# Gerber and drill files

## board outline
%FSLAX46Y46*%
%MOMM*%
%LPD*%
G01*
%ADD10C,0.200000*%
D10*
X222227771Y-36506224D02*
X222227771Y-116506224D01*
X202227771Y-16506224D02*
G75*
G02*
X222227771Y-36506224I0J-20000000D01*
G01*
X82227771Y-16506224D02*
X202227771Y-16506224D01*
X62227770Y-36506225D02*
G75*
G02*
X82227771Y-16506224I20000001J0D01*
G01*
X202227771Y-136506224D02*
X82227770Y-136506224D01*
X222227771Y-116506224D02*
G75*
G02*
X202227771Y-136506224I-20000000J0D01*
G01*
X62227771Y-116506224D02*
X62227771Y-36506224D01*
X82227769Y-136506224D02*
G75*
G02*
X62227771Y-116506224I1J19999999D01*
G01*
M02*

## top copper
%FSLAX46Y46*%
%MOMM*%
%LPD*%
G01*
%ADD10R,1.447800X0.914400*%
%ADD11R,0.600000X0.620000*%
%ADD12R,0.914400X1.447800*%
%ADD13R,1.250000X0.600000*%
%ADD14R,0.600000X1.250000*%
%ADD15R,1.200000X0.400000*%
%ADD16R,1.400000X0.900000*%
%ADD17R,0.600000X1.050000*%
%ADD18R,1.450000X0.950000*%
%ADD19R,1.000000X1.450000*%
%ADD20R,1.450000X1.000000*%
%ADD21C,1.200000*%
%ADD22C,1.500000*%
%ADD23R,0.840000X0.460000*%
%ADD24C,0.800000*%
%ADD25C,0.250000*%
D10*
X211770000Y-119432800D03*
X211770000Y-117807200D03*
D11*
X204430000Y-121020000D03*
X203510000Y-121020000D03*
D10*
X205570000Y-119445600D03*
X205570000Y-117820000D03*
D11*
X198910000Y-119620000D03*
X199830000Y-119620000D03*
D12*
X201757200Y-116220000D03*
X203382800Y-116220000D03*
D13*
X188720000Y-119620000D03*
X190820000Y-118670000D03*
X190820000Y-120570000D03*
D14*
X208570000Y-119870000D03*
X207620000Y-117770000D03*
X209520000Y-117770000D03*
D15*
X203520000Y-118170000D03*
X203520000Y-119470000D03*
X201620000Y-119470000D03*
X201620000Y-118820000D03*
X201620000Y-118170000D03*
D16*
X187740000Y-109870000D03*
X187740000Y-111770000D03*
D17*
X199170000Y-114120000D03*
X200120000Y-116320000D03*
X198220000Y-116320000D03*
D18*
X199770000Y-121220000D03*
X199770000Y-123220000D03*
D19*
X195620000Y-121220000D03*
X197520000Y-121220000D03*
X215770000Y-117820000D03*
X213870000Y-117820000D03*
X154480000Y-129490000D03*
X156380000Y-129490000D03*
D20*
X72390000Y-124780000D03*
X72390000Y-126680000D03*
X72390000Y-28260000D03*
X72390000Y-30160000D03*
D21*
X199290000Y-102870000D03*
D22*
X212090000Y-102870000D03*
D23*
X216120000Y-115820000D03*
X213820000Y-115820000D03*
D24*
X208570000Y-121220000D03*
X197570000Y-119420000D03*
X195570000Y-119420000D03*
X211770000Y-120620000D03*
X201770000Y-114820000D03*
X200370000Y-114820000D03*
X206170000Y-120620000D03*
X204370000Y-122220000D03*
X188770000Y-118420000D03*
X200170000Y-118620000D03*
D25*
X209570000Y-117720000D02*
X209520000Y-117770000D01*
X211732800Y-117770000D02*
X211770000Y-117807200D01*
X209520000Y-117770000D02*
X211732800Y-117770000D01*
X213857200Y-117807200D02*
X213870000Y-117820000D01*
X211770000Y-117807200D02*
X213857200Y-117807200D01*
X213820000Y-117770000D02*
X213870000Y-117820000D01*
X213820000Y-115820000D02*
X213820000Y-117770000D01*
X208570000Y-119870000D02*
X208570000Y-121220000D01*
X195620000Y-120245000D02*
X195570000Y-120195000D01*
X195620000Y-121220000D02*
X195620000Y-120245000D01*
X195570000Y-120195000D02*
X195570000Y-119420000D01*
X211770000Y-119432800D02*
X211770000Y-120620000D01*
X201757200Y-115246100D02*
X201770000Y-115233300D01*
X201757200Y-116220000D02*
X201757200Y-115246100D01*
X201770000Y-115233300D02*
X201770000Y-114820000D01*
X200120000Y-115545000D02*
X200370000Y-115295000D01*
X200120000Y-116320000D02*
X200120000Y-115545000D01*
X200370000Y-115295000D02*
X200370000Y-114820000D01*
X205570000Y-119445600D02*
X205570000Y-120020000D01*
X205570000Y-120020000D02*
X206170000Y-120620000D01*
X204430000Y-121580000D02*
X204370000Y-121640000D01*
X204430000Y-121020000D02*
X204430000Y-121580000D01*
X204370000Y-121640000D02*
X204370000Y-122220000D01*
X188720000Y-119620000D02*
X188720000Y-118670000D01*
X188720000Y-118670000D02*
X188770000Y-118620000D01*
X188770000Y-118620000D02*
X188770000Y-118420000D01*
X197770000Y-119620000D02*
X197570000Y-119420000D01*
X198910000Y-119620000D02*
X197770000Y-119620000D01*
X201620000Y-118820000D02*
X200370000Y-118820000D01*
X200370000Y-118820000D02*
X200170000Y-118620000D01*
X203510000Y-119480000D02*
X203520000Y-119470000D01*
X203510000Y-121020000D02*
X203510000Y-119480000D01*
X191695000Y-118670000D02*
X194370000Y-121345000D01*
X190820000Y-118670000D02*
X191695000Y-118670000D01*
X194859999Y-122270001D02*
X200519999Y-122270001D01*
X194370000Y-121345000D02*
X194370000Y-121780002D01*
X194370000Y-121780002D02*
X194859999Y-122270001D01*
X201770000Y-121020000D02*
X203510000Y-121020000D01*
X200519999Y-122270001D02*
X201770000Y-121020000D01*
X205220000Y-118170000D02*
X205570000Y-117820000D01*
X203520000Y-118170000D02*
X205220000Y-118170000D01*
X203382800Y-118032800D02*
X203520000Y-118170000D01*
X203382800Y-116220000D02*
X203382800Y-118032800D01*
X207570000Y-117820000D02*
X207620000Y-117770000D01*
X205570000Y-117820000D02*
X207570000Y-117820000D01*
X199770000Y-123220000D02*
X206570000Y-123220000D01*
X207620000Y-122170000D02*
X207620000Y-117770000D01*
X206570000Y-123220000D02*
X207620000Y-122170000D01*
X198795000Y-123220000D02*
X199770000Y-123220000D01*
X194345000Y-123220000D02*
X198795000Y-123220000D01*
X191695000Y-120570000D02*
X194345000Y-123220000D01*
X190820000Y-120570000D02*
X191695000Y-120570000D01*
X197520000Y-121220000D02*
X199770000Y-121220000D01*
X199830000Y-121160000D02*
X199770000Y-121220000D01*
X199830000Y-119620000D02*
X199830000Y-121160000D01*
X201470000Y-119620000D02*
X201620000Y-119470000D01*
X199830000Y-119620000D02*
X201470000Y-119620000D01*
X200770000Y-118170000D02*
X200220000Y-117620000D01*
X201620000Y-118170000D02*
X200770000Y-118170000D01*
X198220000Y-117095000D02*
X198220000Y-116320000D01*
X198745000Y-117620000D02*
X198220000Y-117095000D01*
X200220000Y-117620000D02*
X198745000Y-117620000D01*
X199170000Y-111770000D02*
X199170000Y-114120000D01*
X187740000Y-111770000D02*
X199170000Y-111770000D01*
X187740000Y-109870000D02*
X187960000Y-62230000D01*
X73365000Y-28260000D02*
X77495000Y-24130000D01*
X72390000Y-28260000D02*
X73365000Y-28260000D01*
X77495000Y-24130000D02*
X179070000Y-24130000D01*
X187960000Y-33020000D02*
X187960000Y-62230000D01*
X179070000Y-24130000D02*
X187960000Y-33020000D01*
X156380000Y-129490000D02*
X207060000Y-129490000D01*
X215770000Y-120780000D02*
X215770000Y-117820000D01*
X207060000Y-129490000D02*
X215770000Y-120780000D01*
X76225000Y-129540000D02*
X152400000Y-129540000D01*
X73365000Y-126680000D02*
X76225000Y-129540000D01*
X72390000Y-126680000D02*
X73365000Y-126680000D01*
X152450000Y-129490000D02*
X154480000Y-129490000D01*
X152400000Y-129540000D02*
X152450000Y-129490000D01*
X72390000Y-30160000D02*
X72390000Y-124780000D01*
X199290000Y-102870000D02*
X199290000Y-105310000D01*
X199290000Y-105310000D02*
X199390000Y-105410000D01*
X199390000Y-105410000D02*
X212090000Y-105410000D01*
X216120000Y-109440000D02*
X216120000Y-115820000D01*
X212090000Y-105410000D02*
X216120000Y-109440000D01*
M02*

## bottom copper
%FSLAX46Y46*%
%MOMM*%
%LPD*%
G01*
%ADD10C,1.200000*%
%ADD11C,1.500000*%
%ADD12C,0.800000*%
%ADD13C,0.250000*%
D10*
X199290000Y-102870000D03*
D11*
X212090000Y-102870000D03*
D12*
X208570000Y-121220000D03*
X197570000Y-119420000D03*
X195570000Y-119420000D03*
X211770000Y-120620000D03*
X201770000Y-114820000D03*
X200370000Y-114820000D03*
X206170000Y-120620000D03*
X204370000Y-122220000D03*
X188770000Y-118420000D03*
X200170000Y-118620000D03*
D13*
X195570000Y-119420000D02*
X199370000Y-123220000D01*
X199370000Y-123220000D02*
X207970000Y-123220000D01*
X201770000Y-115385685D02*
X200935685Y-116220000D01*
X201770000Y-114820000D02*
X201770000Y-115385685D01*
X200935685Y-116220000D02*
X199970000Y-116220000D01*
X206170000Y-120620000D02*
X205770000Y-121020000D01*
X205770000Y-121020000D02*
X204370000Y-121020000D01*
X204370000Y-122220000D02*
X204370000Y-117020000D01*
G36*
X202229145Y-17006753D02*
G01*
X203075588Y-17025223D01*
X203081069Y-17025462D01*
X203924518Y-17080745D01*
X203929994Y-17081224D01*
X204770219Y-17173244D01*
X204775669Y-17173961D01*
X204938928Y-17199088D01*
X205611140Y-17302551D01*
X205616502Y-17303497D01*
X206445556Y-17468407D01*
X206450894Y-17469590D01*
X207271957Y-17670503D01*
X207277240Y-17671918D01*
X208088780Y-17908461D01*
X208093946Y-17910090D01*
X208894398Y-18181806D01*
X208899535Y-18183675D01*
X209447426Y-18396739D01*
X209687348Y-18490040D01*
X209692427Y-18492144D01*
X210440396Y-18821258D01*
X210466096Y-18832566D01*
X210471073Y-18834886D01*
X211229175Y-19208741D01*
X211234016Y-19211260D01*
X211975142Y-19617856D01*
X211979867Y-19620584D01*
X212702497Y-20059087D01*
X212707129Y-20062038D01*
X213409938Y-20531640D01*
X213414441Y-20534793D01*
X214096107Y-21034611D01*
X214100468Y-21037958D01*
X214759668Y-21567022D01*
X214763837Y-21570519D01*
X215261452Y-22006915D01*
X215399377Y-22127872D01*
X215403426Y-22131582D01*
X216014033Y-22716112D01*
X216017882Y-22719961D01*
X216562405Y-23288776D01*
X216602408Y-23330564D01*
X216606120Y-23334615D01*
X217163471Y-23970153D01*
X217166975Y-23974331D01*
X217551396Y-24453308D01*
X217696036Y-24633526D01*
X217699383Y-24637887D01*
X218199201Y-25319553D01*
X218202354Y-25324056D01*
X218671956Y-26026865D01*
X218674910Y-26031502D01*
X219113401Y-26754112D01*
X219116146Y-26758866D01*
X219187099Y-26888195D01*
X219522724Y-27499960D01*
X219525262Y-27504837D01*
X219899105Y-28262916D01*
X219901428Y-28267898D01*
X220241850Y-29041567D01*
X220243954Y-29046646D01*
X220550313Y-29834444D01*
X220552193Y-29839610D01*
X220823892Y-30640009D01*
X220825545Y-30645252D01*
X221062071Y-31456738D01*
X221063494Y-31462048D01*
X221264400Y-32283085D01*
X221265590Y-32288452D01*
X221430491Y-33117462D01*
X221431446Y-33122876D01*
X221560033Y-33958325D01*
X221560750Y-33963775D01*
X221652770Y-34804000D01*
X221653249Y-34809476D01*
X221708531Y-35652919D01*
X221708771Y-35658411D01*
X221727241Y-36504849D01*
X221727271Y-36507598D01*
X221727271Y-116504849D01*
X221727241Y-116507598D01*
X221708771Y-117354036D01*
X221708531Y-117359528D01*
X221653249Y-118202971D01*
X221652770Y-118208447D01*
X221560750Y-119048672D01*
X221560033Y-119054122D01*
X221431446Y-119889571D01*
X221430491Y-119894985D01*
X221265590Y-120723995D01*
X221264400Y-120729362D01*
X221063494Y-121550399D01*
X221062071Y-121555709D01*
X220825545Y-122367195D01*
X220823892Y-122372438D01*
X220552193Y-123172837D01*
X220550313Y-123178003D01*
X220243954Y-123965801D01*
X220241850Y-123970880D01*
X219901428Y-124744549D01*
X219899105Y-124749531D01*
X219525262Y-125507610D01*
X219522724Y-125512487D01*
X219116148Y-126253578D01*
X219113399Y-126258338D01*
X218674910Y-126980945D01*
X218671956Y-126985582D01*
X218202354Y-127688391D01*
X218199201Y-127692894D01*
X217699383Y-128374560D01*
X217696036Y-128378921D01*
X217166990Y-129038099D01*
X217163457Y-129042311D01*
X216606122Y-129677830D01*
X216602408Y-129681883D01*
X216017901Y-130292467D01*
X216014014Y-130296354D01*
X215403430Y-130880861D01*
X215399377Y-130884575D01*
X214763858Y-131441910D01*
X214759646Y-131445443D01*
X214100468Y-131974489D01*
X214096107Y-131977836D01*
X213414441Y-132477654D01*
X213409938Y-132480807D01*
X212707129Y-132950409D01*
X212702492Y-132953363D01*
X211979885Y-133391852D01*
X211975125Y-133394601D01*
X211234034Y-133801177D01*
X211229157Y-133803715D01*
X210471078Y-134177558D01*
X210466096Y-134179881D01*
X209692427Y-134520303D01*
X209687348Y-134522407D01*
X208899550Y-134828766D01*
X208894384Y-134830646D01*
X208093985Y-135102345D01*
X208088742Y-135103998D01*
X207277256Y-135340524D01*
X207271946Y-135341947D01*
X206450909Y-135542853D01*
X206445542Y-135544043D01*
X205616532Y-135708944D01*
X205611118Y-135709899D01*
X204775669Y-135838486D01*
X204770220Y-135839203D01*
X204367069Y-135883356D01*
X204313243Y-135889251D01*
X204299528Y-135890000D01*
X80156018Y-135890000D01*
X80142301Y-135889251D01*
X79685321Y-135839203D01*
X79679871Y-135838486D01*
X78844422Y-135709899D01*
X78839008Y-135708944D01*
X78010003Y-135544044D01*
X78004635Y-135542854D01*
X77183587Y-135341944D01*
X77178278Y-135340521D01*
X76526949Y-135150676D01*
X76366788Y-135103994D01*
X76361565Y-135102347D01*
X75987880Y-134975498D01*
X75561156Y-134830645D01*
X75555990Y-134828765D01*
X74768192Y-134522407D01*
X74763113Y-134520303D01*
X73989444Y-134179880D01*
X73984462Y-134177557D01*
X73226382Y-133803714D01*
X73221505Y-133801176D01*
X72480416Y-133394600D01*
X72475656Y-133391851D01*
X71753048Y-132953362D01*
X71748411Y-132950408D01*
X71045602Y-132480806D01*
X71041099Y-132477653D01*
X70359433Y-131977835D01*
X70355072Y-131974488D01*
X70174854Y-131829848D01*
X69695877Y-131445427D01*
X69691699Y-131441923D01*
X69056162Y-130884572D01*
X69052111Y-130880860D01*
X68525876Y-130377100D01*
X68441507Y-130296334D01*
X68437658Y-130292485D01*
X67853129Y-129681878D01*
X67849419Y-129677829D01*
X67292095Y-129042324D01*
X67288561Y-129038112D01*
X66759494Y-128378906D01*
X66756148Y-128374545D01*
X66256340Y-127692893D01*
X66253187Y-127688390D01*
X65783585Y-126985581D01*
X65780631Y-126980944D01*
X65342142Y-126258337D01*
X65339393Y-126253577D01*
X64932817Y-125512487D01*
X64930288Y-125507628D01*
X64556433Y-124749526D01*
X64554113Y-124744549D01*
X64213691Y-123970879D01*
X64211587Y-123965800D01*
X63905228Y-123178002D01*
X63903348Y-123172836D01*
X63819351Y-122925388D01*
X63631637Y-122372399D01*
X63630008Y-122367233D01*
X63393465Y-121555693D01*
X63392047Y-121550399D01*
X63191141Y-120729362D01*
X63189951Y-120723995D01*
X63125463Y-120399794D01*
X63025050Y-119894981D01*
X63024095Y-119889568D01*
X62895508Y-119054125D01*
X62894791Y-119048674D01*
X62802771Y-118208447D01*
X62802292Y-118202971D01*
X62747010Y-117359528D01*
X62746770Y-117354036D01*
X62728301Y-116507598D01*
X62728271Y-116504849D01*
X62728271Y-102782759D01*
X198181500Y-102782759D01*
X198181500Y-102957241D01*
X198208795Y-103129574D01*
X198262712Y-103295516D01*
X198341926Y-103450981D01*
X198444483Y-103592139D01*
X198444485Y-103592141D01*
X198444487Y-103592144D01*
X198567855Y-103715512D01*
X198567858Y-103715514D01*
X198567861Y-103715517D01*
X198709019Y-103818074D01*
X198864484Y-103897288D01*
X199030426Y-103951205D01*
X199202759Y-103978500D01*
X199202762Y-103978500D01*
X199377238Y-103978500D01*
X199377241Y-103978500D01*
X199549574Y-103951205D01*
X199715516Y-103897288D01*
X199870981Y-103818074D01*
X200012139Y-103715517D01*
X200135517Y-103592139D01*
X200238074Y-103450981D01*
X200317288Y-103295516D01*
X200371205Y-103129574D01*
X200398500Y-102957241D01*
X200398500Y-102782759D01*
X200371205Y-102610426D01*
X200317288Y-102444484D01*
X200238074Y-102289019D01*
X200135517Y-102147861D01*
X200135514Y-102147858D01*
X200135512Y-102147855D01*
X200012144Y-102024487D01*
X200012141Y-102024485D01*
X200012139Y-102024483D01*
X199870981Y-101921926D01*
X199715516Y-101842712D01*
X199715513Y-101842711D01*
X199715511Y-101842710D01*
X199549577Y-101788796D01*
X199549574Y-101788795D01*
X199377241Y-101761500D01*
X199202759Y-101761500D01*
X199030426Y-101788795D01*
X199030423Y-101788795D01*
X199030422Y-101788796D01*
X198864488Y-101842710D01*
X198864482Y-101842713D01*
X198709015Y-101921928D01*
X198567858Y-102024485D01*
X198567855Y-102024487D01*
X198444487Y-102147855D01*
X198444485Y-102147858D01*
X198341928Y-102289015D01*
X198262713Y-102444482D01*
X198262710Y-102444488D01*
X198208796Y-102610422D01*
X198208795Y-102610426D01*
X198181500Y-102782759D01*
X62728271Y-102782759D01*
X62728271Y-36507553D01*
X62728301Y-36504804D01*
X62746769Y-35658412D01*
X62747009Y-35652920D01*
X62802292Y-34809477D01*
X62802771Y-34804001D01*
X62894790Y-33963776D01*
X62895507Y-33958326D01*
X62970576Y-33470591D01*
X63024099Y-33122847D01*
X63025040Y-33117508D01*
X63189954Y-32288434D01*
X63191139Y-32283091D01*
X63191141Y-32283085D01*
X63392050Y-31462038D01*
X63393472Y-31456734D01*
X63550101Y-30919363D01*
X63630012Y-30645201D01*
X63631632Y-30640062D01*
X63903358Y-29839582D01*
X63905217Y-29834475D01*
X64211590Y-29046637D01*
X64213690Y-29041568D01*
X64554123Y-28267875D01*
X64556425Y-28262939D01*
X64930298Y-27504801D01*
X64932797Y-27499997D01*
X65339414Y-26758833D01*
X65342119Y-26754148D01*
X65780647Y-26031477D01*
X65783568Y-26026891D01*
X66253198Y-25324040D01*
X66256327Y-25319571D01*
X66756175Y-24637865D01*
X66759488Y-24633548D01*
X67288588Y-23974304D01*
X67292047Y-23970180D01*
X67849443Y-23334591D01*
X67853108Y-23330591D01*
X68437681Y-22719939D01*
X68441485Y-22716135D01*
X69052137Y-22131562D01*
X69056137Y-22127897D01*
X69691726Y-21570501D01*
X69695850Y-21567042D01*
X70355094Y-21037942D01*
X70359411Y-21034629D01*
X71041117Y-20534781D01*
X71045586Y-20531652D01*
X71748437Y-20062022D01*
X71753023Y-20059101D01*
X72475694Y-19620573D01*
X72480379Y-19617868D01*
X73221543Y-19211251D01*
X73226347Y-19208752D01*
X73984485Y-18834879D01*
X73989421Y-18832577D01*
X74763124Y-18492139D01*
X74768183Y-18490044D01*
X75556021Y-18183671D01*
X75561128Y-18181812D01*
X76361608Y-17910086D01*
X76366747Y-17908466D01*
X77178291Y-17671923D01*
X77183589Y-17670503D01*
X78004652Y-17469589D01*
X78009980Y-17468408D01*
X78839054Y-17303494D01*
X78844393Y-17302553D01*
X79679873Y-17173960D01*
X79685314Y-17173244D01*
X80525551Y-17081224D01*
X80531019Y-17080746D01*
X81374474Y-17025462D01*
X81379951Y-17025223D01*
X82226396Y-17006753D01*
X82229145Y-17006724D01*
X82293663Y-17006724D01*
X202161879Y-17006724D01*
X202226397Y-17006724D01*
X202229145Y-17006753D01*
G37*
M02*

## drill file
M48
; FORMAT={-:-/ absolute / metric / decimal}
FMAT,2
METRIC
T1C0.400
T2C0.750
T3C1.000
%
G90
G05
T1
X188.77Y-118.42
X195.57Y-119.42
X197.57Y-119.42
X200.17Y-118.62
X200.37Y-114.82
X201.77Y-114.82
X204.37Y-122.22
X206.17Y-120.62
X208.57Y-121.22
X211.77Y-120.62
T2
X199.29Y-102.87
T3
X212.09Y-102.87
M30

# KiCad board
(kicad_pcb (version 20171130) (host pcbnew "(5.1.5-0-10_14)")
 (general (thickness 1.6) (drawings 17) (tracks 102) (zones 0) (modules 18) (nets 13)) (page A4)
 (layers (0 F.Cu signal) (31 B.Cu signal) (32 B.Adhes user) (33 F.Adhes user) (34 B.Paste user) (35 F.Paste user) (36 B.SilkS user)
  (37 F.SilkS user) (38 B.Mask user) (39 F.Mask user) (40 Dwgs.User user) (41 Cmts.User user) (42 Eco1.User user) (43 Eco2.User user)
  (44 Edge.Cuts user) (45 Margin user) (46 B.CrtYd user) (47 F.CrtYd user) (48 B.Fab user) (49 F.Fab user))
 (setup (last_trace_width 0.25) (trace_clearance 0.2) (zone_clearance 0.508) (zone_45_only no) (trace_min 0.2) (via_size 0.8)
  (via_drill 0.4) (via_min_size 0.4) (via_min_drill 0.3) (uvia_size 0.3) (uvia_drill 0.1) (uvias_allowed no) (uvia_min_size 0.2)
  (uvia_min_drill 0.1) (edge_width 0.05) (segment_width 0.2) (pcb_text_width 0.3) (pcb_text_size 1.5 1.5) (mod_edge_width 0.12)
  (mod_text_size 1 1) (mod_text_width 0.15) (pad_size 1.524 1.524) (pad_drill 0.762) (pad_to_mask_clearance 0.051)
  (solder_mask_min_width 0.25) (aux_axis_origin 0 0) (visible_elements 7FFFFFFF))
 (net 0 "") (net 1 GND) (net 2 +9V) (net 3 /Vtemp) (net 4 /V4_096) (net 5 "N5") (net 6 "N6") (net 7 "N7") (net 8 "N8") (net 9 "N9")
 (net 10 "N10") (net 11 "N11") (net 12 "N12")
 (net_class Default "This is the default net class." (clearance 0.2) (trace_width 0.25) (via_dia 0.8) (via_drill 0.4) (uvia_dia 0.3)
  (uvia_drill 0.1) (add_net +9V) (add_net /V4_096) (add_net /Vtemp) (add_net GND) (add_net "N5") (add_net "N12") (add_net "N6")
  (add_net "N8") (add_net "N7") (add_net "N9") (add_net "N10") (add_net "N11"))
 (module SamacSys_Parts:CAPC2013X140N (layer F.Cu) (at 211.77 118.62 270)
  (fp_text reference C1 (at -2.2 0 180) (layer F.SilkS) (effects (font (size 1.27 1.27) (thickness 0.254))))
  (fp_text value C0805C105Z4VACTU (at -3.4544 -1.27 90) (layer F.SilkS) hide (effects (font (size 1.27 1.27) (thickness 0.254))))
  (pad 2 smd rect (at 0.8128 0 270) (size 0.9144 1.4478) (layers F.Cu F.Paste F.Mask) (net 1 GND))
  (pad 1 smd rect (at -0.8128 0 270) (size 0.9144 1.4478) (layers F.Cu F.Paste F.Mask) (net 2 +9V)))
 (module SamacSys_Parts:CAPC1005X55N (layer F.Cu) (at 203.97 121.02)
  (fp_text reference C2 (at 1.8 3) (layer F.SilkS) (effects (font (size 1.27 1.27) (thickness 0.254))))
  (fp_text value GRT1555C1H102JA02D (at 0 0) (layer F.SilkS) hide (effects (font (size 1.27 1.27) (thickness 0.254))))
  (pad 2 smd rect (at 0.46 0) (size 0.6 0.62) (layers F.Cu F.Paste F.Mask) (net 1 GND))
  (pad 1 smd rect (at -0.46 0) (size 0.6 0.62) (layers F.Cu F.Paste F.Mask) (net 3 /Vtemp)))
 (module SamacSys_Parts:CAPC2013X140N (layer F.Cu) (at 205.57 118.6328 270)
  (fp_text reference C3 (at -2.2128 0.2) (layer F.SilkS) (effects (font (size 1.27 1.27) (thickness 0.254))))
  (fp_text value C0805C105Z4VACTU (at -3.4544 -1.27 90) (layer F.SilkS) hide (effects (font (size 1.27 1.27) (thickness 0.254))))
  (pad 2 smd rect (at 0.8128 0 270) (size 0.9144 1.4478) (layers F.Cu F.Paste F.Mask) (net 1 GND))
  (pad 1 smd rect (at -0.8128 0 270) (size 0.9144 1.4478) (layers F.Cu F.Paste F.Mask) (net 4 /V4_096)))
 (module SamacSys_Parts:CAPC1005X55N (layer F.Cu) (at 199.37 119.62 180)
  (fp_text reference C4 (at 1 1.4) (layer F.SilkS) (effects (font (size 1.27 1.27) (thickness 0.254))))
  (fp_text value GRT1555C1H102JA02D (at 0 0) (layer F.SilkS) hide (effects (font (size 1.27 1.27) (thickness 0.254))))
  (pad 2 smd rect (at 0.46 0 180) (size 0.6 0.62) (layers F.Cu F.Paste F.Mask) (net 1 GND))
  (pad 1 smd rect (at -0.46 0 180) (size 0.6 0.62) (layers F.Cu F.Paste F.Mask) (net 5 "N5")))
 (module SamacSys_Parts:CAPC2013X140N (layer F.Cu) (at 202.57 116.22 180)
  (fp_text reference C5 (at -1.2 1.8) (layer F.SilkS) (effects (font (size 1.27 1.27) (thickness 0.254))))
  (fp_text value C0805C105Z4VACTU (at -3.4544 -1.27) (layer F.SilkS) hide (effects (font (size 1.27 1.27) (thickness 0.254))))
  (pad 2 smd rect (at 0.8128 0 180) (size 0.9144 1.4478) (layers F.Cu F.Paste F.Mask) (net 1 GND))
  (pad 1 smd rect (at -0.8128 0 180) (size 0.9144 1.4478) (layers F.Cu F.Paste F.Mask) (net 4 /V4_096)))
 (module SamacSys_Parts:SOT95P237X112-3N (layer F.Cu) (at 189.77 119.62 180)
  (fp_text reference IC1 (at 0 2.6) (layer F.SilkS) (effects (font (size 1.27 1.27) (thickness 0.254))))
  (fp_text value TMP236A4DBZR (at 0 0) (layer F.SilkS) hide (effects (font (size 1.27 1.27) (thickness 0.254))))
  (pad 3 smd rect (at 1.05 0 270) (size 0.6 1.25) (layers F.Cu F.Paste F.Mask) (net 1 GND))
  (pad 2 smd rect (at -1.05 0.95 270) (size 0.6 1.25) (layers F.Cu F.Paste F.Mask) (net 3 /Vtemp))
  (pad 1 smd rect (at -1.05 -0.95 270) (size 0.6 1.25) (layers F.Cu F.Paste F.Mask) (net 4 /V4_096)))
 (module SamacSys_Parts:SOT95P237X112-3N (layer F.Cu) (at 208.57 118.82 270)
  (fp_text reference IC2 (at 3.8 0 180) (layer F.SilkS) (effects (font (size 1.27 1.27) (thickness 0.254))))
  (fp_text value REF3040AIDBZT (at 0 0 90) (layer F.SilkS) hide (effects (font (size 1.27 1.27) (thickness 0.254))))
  (pad 3 smd rect (at 1.05 0) (size 0.6 1.25) (layers F.Cu F.Paste F.Mask) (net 1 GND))
  (pad 2 smd rect (at -1.05 0.95) (size 0.6 1.25) (layers F.Cu F.Paste F.Mask) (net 4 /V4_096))
  (pad 1 smd rect (at -1.05 -0.95) (size 0.6 1.25) (layers F.Cu F.Paste F.Mask) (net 2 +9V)))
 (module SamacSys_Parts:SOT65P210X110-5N (layer F.Cu) (at 202.57 118.82)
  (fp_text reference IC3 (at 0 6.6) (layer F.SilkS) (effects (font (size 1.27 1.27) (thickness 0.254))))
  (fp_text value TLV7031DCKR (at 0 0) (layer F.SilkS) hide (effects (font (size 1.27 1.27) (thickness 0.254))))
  (pad 5 smd rect (at 0.95 -0.65 90) (size 0.4 1.2) (layers F.Cu F.Paste F.Mask) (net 4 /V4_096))
  (pad 4 smd rect (at 0.95 0.65 90) (size 0.4 1.2) (layers F.Cu F.Paste F.Mask) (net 3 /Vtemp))
  (pad 3 smd rect (at -0.95 0.65 90) (size 0.4 1.2) (layers F.Cu F.Paste F.Mask) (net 5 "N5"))
  (pad 2 smd rect (at -0.95 0 90) (size 0.4 1.2) (layers F.Cu F.Paste F.Mask) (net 1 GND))
  (pad 1 smd rect (at -0.95 -0.65 90) (size 0.4 1.2) (layers F.Cu F.Paste F.Mask) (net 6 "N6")))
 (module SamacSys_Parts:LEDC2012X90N (layer F.Cu) (at 187.74 110.82 90)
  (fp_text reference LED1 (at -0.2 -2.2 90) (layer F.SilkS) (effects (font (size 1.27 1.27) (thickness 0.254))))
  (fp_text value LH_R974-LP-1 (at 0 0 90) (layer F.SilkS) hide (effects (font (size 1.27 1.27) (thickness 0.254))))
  (pad 2 smd rect (at 0.95 0 90) (size 0.9 1.4) (layers F.Cu F.Paste F.Mask) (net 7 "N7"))
  (pad 1 smd rect (at -0.95 0 90) (size 0.9 1.4) (layers F.Cu F.Paste F.Mask) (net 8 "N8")))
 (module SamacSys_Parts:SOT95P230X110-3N (layer F.Cu) (at 199.17 115.22 90)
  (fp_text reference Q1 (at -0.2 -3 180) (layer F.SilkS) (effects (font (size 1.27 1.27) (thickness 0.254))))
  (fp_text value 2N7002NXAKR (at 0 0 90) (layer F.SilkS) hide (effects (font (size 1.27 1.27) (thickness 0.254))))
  (pad 3 smd rect (at 1.1 0 180) (size 0.6 1.05) (layers F.Cu F.Paste F.Mask) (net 8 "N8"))
  (pad 2 smd rect (at -1.1 0.95 180) (size 0.6 1.05) (layers F.Cu F.Paste F.Mask) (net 1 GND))
  (pad 1 smd rect (at -1.1 -0.95 180) (size 0.6 1.05) (layers F.Cu F.Paste F.Mask) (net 6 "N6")))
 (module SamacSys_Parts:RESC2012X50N (layer F.Cu) (at 199.77 122.22 90)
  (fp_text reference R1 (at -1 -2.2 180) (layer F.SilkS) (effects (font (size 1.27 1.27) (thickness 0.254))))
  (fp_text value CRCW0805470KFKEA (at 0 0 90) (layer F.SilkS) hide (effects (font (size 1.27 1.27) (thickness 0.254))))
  (pad 2 smd rect (at 1 0 90) (size 0.95 1.45) (layers F.Cu F.Paste F.Mask) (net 5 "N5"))
  (pad 1 smd rect (at -1 0 90) (size 0.95 1.45) (layers F.Cu F.Paste F.Mask) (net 4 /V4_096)))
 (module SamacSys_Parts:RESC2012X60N (layer F.Cu) (at 196.57 121.22 180)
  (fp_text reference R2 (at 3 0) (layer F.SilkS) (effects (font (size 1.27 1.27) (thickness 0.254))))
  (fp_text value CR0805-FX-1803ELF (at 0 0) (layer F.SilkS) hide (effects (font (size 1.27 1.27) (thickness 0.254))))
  (pad 2 smd rect (at 0.95 0 180) (size 1 1.45) (layers F.Cu F.Paste F.Mask) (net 1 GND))
  (pad 1 smd rect (at -0.95 0 180) (size 1 1.45) (layers F.Cu F.Paste F.Mask) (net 5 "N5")))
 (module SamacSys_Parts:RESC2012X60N (layer F.Cu) (at 214.82 117.82)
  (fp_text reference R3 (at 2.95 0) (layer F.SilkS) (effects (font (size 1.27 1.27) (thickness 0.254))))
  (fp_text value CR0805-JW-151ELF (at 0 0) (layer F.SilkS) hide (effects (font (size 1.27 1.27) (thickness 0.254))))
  (pad 2 smd rect (at 0.95 0) (size 1 1.45) (layers F.Cu F.Paste F.Mask) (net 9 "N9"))
  (pad 1 smd rect (at -0.95 0) (size 1 1.45) (layers F.Cu F.Paste F.Mask) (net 2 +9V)))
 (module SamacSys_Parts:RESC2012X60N (layer F.Cu) (at 155.43 129.49 180)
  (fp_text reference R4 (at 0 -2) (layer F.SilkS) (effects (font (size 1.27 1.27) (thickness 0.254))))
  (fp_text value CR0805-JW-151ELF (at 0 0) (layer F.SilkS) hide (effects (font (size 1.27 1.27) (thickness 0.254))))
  (pad 2 smd rect (at 0.95 0 180) (size 1 1.45) (layers F.Cu F.Paste F.Mask) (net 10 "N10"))
  (pad 1 smd rect (at -0.95 0 180) (size 1 1.45) (layers F.Cu F.Paste F.Mask) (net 9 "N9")))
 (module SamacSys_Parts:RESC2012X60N (layer F.Cu) (at 72.39 125.73 90)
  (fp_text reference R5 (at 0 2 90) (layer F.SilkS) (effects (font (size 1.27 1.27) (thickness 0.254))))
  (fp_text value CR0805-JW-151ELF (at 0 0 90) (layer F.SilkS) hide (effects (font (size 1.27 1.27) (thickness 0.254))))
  (pad 2 smd rect (at 0.95 0 90) (size 1 1.45) (layers F.Cu F.Paste F.Mask) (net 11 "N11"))
  (pad 1 smd rect (at -0.95 0 90) (size 1 1.45) (layers F.Cu F.Paste F.Mask) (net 10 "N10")))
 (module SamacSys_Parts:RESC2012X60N (layer F.Cu) (at 72.39 29.21 90)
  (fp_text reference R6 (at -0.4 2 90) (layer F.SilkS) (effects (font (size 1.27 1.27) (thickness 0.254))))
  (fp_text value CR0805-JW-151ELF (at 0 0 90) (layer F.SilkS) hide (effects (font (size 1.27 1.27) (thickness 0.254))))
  (pad 2 smd rect (at 0.95 0 90) (size 1 1.45) (layers F.Cu F.Paste F.Mask) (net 7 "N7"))
  (pad 1 smd rect (at -0.95 0 90) (size 1 1.45) (layers F.Cu F.Paste F.Mask) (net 11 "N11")))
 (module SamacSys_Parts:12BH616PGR (layer F.Cu) (at 212.09 102.87 270)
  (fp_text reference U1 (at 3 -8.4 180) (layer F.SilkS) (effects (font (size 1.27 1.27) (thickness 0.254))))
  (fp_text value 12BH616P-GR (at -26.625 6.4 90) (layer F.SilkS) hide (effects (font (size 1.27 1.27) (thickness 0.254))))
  (pad 2 thru_hole circle (at 0 12.8 270) (size 1.2 1.2) (drill 0.75) (layers *.Cu *.Mask) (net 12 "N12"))
  (pad 1 thru_hole circle (at 0 0 270) (size 1.5 1.5) (drill 1) (layers *.Cu *.Mask) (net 1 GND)))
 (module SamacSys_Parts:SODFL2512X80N (layer F.Cu) (at 214.97 115.82)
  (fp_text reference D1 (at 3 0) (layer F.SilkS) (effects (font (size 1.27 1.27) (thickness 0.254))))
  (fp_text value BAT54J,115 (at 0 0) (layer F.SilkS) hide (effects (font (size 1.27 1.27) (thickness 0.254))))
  (pad 2 smd rect (at 1.15 0 90) (size 0.46 0.84) (layers F.Cu F.Paste F.Mask) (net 12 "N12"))
  (pad 1 smd rect (at -1.15 0 90) (size 0.46 0.84) (layers F.Cu F.Paste F.Mask) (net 2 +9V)))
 (gr_line (start 222.227771 36.506224) (end 222.227771 116.506224) (layer Edge.Cuts) (width 0.2))
 (gr_arc (start 202.227771 36.506224) (end 222.227771 36.506224) (angle -90) (layer Edge.Cuts) (width 0.2))
 (gr_line (start 82.227771 16.506224) (end 202.227771 16.506224) (layer Edge.Cuts) (width 0.2))
 (gr_arc (start 82.227771 36.506225) (end 82.227771 16.506224) (angle -90) (layer Edge.Cuts) (width 0.2))
 (gr_line (start 202.227771 136.506224) (end 82.22777 136.506224) (layer Edge.Cuts) (width 0.2))
 (gr_arc (start 202.227771 116.506224) (end 202.227771 136.506224) (angle -90) (layer Edge.Cuts) (width 0.2))
 (gr_line (start 62.227771 116.506224) (end 62.227771 36.506224) (layer Edge.Cuts) (width 0.2))
 (gr_arc (start 82.22777 116.506225) (end 62.227771 116.506224) (angle -90) (layer Edge.Cuts) (width 0.2))
 (segment (start 209.57 117.72) (end 209.52 117.77) (width 0.25) (layer F.Cu) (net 2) (status 30))
 (segment (start 211.7328 117.77) (end 211.77 117.8072) (width 0.25) (layer F.Cu) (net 2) (status 30))
 (segment (start 209.52 117.77) (end 211.7328 117.77) (width 0.25) (layer F.Cu) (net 2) (status 30))
 (segment (start 213.8572 117.8072) (end 213.87 117.82) (width 0.25) (layer F.Cu) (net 2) (status 30))
 (segment (start 211.77 117.8072) (end 213.8572 117.8072) (width 0.25) (layer F.Cu) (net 2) (status 30))
 (segment (start 213.82 117.77) (end 213.87 117.82) (width 0.25) (layer F.Cu) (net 2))
 (segment (start 213.82 115.82) (end 213.82 117.77) (width 0.25) (layer F.Cu) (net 2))
 (segment (start 208.57 119.87) (end 208.57 121.22) (width 0.25) (layer F.Cu) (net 1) (status 10))
 (via (at 208.57 121.22) (size 0.8) (drill 0.4) (layers F.Cu B.Cu) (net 1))
 (via (at 197.57 119.42) (size 0.8) (drill 0.4) (layers F.Cu B.Cu) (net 1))
 (segment (start 195.62 120.245) (end 195.57 120.195) (width 0.25) (layer F.Cu) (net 1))
 (segment (start 195.62 121.22) (end 195.62 120.245) (width 0.25) (layer F.Cu) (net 1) (status 10))
 (via (at 195.57 119.42) (size 0.8) (drill 0.4) (layers F.Cu B.Cu) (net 1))
 (segment (start 195.57 120.195) (end 195.57 119.42) (width 0.25) (layer F.Cu) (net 1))
 (segment (start 195.57 119.42) (end 199.37 123.22) (width 0.25) (layer B.Cu) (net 1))
 (segment (start 199.37 123.22) (end 207.97 123.22) (width 0.25) (layer B.Cu) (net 1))
 (segment (start 211.77 119.4328) (end 211.77 120.62) (width 0.25) (layer F.Cu) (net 1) (status 10))
 (via (at 211.77 120.62) (size 0.8) (drill 0.4) (layers F.Cu B.Cu) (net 1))
 (segment (start 201.7572 115.2461) (end 201.77 115.2333) (width 0.25) (layer F.Cu) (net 1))
 (segment (start 201.7572 116.22) (end 201.7572 115.2461) (width 0.25) (layer F.Cu) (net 1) (status 10))
 (via (at 201.77 114.82) (size 0.8) (drill 0.4) (layers F.Cu B.Cu) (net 1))
 (segment (start 201.77 115.2333) (end 201.77 114.82) (width 0.25) (layer F.Cu) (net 1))
 (segment (start 201.77 115.385685) (end 200.935685 116.22) (width 0.25) (layer B.Cu) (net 1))
 (segment (start 201.77 114.82) (end 201.77 115.385685) (width 0.25) (layer B.Cu) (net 1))
 (segment (start 200.935685 116.22) (end 199.97 116.22) (width 0.25) (layer B.Cu) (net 1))
 (segment (start 200.12 115.545) (end 200.37 115.295) (width 0.25) (layer F.Cu) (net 1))
 (segment (start 200.12 116.32) (end 200.12 115.545) (width 0.25) (layer F.Cu) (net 1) (status 10))
 (via (at 200.37 114.82) (size 0.8) (drill 0.4) (layers F.Cu B.Cu) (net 1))
 (segment (start 200.37 115.295) (end 200.37 114.82) (width 0.25) (layer F.Cu) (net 1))
 (via (at 206.17 120.62) (size 0.8) (drill 0.4) (layers F.Cu B.Cu) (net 1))
 (segment (start 205.57 119.4456) (end 205.57 120.02) (width 0.25) (layer F.Cu) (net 1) (status 10))
 (segment (start 205.57 120.02) (end 206.17 120.62) (width 0.25) (layer F.Cu) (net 1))
 (segment (start 206.17 120.62) (end 205.77 121.02) (width 0.25) (layer B.Cu) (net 1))
 (segment (start 205.77 121.02) (end 204.37 121.02) (width 0.25) (layer B.Cu) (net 1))
 (segment (start 204.43 121.58) (end 204.37 121.64) (width 0.25) (layer F.Cu) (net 1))
 (segment (start 204.43 121.02) (end 204.43 121.58) (width 0.25) (layer F.Cu) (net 1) (status 10))
 (via (at 204.37 122.22) (size 0.8) (drill 0.4) (layers F.Cu B.Cu) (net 1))
 (segment (start 204.37 121.64) (end 204.37 122.22) (width 0.25) (layer F.Cu) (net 1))
 (segment (start 204.37 122.22) (end 204.37 117.02) (width 0.25) (layer B.Cu) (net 1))
 (segment (start 188.72 119.62) (end 188.72 118.67) (width 0.25) (layer F.Cu) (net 1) (status 10))
 (segment (start 188.72 118.67) (end 188.77 118.62) (width 0.25) (layer F.Cu) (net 1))
 (via (at 188.77 118.42) (size 0.8) (drill 0.4) (layers F.Cu B.Cu) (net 1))
 (segment (start 188.77 118.62) (end 188.77 118.42) (width 0.25) (layer F.Cu) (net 1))
 (segment (start 197.77 119.62) (end 197.57 119.42) (width 0.25) (layer F.Cu) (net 1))
 (segment (start 198.91 119.62) (end 197.77 119.62) (width 0.25) (layer F.Cu) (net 1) (status 10))
 (via (at 200.17 118.62) (size 0.8) (drill 0.4) (layers F.Cu B.Cu) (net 1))
 (segment (start 201.62 118.82) (end 200.37 118.82) (width 0.25) (layer F.Cu) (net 1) (status 10))
 (segment (start 200.37 118.82) (end 200.17 118.62) (width 0.25) (layer F.Cu) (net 1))
 (segment (start 203.51 119.48) (end 203.52 119.47) (width 0.25) (layer F.Cu) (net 3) (status 30))
 (segment (start 203.51 121.02) (end 203.51 119.48) (width 0.25) (layer F.Cu) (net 3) (status 30))
 (segment (start 191.695 118.67) (end 194.37 121.345) (width 0.25) (layer F.Cu) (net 3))
 (segment (start 190.82 118.67) (end 191.695 118.67) (width 0.25) (layer F.Cu) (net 3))
 (segment (start 194.859999 122.270001) (end 200.519999 122.270001) (width 0.25) (layer F.Cu) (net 3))
 (segment (start 194.37 121.345) (end 194.37 121.780002) (width 0.25) (layer F.Cu) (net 3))
 (segment (start 194.37 121.780002) (end 194.859999 122.270001) (width 0.25) (layer F.Cu) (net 3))
 (segment (start 201.77 121.02) (end 203.51 121.02) (width 0.25) (layer F.Cu) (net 3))
 (segment (start 200.519999 122.270001) (end 201.77 121.02) (width 0.25) (layer F.Cu) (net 3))
 (segment (start 205.22 118.17) (end 205.57 117.82) (width 0.25) (layer F.Cu) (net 4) (status 30))
 (segment (start 203.52 118.17) (end 205.22 118.17) (width 0.25) (layer F.Cu) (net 4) (status 30))
 (segment (start 203.3828 118.0328) (end 203.52 118.17) (width 0.25) (layer F.Cu) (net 4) (status 30))
 (segment (start 203.3828 116.22) (end 203.3828 118.0328) (width 0.25) (layer F.Cu) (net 4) (status 30))
 (segment (start 207.57 117.82) (end 207.62 117.77) (width 0.25) (layer F.Cu) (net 4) (status 30))
 (segment (start 205.57 117.82) (end 207.57 117.82) (width 0.25) (layer F.Cu) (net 4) (status 30))
 (segment (start 199.77 123.22) (end 206.57 123.22) (width 0.25) (layer F.Cu) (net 4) (status 10))
 (segment (start 207.62 122.17) (end 207.62 117.77) (width 0.25) (layer F.Cu) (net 4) (status 20))
 (segment (start 206.57 123.22) (end 207.62 122.17) (width 0.25) (layer F.Cu) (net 4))
 (segment (start 198.795 123.22) (end 199.77 123.22) (width 0.25) (layer F.Cu) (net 4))
 (segment (start 194.345 123.22) (end 198.795 123.22) (width 0.25) (layer F.Cu) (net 4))
 (segment (start 191.695 120.57) (end 194.345 123.22) (width 0.25) (layer F.Cu) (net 4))
 (segment (start 190.82 120.57) (end 191.695 120.57) (width 0.25) (layer F.Cu) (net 4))
 (segment (start 197.52 121.22) (end 199.77 121.22) (width 0.25) (layer F.Cu) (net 5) (status 30))
 (segment (start 199.83 121.16) (end 199.77 121.22) (width 0.25) (layer F.Cu) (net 5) (status 30))
 (segment (start 199.83 119.62) (end 199.83 121.16) (width 0.25) (layer F.Cu) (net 5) (status 30))
 (segment (start 201.47 119.62) (end 201.62 119.47) (width 0.25) (layer F.Cu) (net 5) (status 30))
 (segment (start 199.83 119.62) (end 201.47 119.62) (width 0.25) (layer F.Cu) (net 5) (status 30))
 (segment (start 200.77 118.17) (end 200.22 117.62) (width 0.25) (layer F.Cu) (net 6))
 (segment (start 201.62 118.17) (end 200.77 118.17) (width 0.25) (layer F.Cu) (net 6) (status 10))
 (segment (start 198.22 117.095) (end 198.22 116.32) (width 0.25) (layer F.Cu) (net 6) (status 20))
 (segment (start 198.745 117.62) (end 198.22 117.095) (width 0.25) (layer F.Cu) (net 6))
 (segment (start 200.22 117.62) (end 198.745 117.62) (width 0.25) (layer F.Cu) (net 6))
 (segment (start 199.17 111.77) (end 199.17 114.12) (width 0.25) (layer F.Cu) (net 8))
 (segment (start 187.74 111.77) (end 199.17 111.77) (width 0.25) (layer F.Cu) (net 8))
 (segment (start 187.74 109.87) (end 187.96 62.23) (width 0.25) (layer F.Cu) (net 7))
 (segment (start 73.365 28.26) (end 77.495 24.13) (width 0.25) (layer F.Cu) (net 7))
 (segment (start 72.39 28.26) (end 73.365 28.26) (width 0.25) (layer F.Cu) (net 7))
 (segment (start 77.495 24.13) (end 179.07 24.13) (width 0.25) (layer F.Cu) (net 7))
 (segment (start 187.96 33.02) (end 187.96 62.23) (width 0.25) (layer F.Cu) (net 7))
 (segment (start 179.07 24.13) (end 187.96 33.02) (width 0.25) (layer F.Cu) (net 7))
 (segment (start 156.38 129.49) (end 207.06 129.49) (width 0.25) (layer F.Cu) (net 9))
 (segment (start 215.77 120.78) (end 215.77 117.82) (width 0.25) (layer F.Cu) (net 9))
 (segment (start 207.06 129.49) (end 215.77 120.78) (width 0.25) (layer F.Cu) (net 9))
 (segment (start 76.225 129.54) (end 152.4 129.54) (width 0.25) (layer F.Cu) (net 10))
 (segment (start 73.365 126.68) (end 76.225 129.54) (width 0.25) (layer F.Cu) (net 10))
 (segment (start 72.39 126.68) (end 73.365 126.68) (width 0.25) (layer F.Cu) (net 10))
 (segment (start 152.45 129.49) (end 154.48 129.49) (width 0.25) (layer F.Cu) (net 10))
 (segment (start 152.4 129.54) (end 152.45 129.49) (width 0.25) (layer F.Cu) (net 10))
 (segment (start 72.39 30.16) (end 72.39 124.78) (width 0.25) (layer F.Cu) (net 11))
 (segment (start 199.29 102.87) (end 199.29 105.31) (width 0.25) (layer F.Cu) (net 12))
 (segment (start 199.29 105.31) (end 199.39 105.41) (width 0.25) (layer F.Cu) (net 12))
 (segment (start 199.39 105.41) (end 212.09 105.41) (width 0.25) (layer F.Cu) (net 12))
 (segment (start 216.12 109.44) (end 216.12 115.82) (width 0.25) (layer F.Cu) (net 12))
 (segment (start 212.09 105.41) (end 216.12 109.44) (width 0.25) (layer F.Cu) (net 12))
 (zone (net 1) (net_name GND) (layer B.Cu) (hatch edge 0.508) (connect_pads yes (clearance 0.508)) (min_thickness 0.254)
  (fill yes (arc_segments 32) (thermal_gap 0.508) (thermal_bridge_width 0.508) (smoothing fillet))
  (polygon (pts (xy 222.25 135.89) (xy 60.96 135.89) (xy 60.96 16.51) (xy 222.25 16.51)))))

